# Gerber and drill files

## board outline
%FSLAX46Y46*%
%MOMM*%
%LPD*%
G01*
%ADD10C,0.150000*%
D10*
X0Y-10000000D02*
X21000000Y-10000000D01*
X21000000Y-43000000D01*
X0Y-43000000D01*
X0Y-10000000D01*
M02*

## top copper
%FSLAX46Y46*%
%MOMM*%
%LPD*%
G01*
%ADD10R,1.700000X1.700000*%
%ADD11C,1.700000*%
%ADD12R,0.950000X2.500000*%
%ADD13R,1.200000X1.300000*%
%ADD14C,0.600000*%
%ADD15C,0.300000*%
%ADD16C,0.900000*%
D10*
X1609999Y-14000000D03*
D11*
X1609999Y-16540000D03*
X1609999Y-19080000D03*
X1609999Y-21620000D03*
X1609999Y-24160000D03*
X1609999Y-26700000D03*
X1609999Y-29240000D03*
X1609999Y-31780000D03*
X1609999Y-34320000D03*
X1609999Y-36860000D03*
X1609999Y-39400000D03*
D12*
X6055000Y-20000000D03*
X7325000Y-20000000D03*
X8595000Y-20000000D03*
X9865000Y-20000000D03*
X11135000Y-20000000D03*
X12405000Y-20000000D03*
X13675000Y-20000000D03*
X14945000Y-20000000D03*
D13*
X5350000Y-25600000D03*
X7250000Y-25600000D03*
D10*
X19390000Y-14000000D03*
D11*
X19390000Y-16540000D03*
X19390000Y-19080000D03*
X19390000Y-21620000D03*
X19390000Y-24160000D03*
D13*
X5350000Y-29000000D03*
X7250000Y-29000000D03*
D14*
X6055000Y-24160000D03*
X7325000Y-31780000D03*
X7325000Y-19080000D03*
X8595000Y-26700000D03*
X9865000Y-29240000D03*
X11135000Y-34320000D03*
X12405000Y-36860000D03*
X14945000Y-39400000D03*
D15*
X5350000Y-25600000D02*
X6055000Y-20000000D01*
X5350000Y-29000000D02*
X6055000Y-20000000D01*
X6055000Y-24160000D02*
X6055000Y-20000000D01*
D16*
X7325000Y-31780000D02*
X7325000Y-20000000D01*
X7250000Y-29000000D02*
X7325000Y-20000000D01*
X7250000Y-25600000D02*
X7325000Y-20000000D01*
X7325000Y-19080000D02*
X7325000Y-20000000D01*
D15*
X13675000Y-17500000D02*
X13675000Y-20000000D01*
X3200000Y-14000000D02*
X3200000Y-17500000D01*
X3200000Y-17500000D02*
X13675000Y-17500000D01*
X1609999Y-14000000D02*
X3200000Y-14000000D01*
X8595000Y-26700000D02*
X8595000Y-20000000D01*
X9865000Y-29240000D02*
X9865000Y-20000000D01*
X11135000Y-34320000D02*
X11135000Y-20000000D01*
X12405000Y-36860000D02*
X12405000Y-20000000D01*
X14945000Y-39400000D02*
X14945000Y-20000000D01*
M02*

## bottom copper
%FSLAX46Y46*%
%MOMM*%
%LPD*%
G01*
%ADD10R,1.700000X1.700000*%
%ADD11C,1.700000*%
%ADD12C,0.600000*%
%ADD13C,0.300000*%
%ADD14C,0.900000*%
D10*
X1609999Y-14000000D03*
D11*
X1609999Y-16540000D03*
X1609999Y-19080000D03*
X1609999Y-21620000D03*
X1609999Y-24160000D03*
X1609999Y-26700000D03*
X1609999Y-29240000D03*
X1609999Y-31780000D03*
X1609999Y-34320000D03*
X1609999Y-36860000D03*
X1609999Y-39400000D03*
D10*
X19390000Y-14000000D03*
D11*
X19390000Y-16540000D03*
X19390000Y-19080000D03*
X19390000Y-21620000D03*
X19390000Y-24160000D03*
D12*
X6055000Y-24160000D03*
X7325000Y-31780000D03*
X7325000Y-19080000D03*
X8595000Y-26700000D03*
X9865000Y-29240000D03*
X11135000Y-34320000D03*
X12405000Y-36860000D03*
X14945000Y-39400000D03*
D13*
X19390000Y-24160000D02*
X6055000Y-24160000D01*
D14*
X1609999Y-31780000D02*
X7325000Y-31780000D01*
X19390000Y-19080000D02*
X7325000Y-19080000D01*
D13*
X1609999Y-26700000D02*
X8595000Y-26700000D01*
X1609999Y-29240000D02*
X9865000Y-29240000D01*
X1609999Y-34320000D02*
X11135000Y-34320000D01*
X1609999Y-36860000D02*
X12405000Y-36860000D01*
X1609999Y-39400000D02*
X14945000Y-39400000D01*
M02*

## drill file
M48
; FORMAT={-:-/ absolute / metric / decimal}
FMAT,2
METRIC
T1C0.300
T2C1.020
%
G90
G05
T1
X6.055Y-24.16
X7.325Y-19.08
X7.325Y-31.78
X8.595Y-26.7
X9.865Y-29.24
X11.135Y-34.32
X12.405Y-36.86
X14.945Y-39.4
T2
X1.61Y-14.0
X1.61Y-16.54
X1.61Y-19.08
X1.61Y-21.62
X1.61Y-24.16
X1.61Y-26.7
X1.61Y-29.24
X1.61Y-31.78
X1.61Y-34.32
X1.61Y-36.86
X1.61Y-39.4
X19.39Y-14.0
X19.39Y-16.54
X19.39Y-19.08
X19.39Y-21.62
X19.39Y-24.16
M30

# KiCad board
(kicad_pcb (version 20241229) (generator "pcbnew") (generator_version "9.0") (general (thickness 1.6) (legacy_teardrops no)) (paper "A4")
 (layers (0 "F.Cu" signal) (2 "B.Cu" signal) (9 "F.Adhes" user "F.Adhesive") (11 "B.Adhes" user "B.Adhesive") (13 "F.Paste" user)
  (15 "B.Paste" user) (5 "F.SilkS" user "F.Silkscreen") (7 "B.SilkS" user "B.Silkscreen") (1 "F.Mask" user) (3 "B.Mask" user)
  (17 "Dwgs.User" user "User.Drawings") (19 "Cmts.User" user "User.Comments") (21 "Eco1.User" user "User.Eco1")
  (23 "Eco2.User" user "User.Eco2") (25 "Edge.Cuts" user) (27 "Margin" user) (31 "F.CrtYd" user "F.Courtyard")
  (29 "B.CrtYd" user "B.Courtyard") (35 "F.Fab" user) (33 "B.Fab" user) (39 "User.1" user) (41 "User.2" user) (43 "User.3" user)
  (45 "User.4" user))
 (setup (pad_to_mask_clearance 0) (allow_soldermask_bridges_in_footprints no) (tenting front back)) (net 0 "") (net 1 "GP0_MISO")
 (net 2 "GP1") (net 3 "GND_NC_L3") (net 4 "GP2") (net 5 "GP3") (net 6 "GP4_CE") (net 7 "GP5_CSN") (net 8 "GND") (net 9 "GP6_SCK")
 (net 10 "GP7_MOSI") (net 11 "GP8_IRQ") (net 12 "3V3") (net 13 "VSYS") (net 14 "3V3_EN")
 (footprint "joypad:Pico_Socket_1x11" (layer "F.Cu") (at 1.609999 14)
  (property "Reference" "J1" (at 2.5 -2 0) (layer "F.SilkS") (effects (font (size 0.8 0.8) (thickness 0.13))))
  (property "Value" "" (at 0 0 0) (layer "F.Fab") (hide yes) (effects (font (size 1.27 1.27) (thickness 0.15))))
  (pad "1" thru_hole rect (at 0 0) (size 1.7 1.7) (drill 1.02) (layers "*.Cu" "*.Mask") (remove_unused_layers no) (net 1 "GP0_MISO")
   (thermal_bridge_angle 45))
  (pad "2" thru_hole circle (at 0 2.54) (size 1.7 1.7) (drill 1.02) (layers "*.Cu" "*.Mask") (remove_unused_layers no) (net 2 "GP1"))
  (pad "3" thru_hole circle (at 0 5.08) (size 1.7 1.7) (drill 1.02) (layers "*.Cu" "*.Mask") (remove_unused_layers no) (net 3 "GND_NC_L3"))
  (pad "4" thru_hole circle (at 0 7.62) (size 1.7 1.7) (drill 1.02) (layers "*.Cu" "*.Mask") (remove_unused_layers no) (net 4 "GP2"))
  (pad "5" thru_hole circle (at 0 10.16) (size 1.7 1.7) (drill 1.02) (layers "*.Cu" "*.Mask") (remove_unused_layers no) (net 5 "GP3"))
  (pad "6" thru_hole circle (at 0 12.7) (size 1.7 1.7) (drill 1.02) (layers "*.Cu" "*.Mask") (remove_unused_layers no) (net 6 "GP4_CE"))
  (pad "7" thru_hole circle (at 0 15.24) (size 1.7 1.7) (drill 1.02) (layers "*.Cu" "*.Mask") (remove_unused_layers no) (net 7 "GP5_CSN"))
  (pad "8" thru_hole circle (at 0 17.78) (size 1.7 1.7) (drill 1.02) (layers "*.Cu" "*.Mask") (remove_unused_layers no) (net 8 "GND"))
  (pad "9" thru_hole circle (at 0 20.32) (size 1.7 1.7) (drill 1.02) (layers "*.Cu" "*.Mask") (remove_unused_layers no) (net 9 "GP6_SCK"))
  (pad "10" thru_hole circle (at 0 22.86) (size 1.7 1.7) (drill 1.02) (layers "*.Cu" "*.Mask") (remove_unused_layers no) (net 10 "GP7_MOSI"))
  (pad "11" thru_hole circle (at 0 25.4) (size 1.7 1.7) (drill 1.02) (layers "*.Cu" "*.Mask") (remove_unused_layers no) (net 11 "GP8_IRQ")))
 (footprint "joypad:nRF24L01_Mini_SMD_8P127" (layer "F.Cu") (at 10.5 20)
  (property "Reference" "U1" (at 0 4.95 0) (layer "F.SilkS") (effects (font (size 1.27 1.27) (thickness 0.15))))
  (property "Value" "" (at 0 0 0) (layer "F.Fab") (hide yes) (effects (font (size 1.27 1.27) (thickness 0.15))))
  (pad "1" smd rect (at -4.445 0) (size 0.95 2.5) (layers "F.Cu" "F.Mask" "F.Paste") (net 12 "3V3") (thermal_bridge_angle 45))
  (pad "2" smd rect (at -3.175 0) (size 0.95 2.5) (layers "F.Cu" "F.Mask" "F.Paste") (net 8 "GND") (thermal_bridge_angle 45))
  (pad "3" smd rect (at -1.905 0) (size 0.95 2.5) (layers "F.Cu" "F.Mask" "F.Paste") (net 6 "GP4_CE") (thermal_bridge_angle 45))
  (pad "4" smd rect (at -0.635 0) (size 0.95 2.5) (layers "F.Cu" "F.Mask" "F.Paste") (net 7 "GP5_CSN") (thermal_bridge_angle 45))
  (pad "5" smd rect (at 0.635 0) (size 0.95 2.5) (layers "F.Cu" "F.Mask" "F.Paste") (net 9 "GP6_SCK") (thermal_bridge_angle 45))
  (pad "6" smd rect (at 1.905 0) (size 0.95 2.5) (layers "F.Cu" "F.Mask" "F.Paste") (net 10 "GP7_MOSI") (thermal_bridge_angle 45))
  (pad "7" smd rect (at 3.175 0) (size 0.95 2.5) (layers "F.Cu" "F.Mask" "F.Paste") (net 1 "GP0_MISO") (thermal_bridge_angle 45))
  (pad "8" smd rect (at 4.445 0) (size 0.95 2.5) (layers "F.Cu" "F.Mask" "F.Paste") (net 11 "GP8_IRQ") (thermal_bridge_angle 45))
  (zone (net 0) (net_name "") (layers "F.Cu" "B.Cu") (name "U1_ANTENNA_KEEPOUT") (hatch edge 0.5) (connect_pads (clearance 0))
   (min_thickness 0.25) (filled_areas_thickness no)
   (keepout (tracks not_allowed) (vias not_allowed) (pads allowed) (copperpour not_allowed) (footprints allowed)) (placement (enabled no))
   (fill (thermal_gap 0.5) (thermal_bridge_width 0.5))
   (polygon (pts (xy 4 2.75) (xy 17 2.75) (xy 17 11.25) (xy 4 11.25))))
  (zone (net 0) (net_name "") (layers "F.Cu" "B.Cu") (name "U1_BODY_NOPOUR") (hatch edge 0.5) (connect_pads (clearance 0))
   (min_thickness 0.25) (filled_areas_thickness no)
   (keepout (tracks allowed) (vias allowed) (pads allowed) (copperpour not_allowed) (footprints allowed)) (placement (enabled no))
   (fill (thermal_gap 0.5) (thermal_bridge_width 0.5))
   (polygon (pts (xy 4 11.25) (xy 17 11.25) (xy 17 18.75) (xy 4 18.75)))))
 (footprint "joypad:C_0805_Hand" (layer "F.Cu") (at 6.3 25.6)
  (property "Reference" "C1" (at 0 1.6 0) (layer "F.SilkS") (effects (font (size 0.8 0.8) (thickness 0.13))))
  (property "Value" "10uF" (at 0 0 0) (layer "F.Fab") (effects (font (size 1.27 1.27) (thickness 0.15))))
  (pad "1" smd rect (at -0.95 0) (size 1.2 1.3) (layers "F.Cu" "F.Mask" "F.Paste") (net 12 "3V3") (thermal_bridge_angle 45))
  (pad "2" smd rect (at 0.95 0) (size 1.2 1.3) (layers "F.Cu" "F.Mask" "F.Paste") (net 8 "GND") (thermal_bridge_angle 45)))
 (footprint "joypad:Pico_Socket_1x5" (layer "F.Cu") (at 19.39 14)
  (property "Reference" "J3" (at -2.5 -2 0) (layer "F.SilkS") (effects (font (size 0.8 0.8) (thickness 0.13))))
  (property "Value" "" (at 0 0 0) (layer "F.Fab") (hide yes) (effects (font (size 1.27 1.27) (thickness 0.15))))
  (pad "1" thru_hole rect (at 0 0) (size 1.7 1.7) (drill 1.02) (layers "*.Cu" "*.Mask") (remove_unused_layers no) (thermal_bridge_angle 45))
  (pad "2" thru_hole circle (at 0 2.54) (size 1.7 1.7) (drill 1.02) (layers "*.Cu" "*.Mask") (remove_unused_layers no) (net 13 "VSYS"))
  (pad "3" thru_hole circle (at 0 5.08) (size 1.7 1.7) (drill 1.02) (layers "*.Cu" "*.Mask") (remove_unused_layers no) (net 8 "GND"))
  (pad "4" thru_hole circle (at 0 7.62) (size 1.7 1.7) (drill 1.02) (layers "*.Cu" "*.Mask") (remove_unused_layers no) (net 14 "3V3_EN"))
  (pad "5" thru_hole circle (at 0 10.16) (size 1.7 1.7) (drill 1.02) (layers "*.Cu" "*.Mask") (remove_unused_layers no) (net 12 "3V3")))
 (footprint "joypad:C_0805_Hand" (layer "F.Cu") (at 6.3 29)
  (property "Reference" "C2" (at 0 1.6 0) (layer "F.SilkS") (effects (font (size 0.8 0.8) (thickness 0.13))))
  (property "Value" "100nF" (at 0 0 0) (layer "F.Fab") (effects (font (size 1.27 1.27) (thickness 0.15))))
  (pad "1" smd rect (at -0.95 0) (size 1.2 1.3) (layers "F.Cu" "F.Mask" "F.Paste") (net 12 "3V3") (thermal_bridge_angle 45))
  (pad "2" smd rect (at 0.95 0) (size 1.2 1.3) (layers "F.Cu" "F.Mask" "F.Paste") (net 8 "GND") (thermal_bridge_angle 45)))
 (gr_rect (start 0 10) (end 21 43) (stroke (width 0.15) (type default)) (fill no) (layer "Edge.Cuts"))
 (segment (start 5.35 25.6) (end 6.055 20) (width 0.3) (layer "F.Cu") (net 12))
 (segment (start 5.35 29) (end 6.055 20) (width 0.3) (layer "F.Cu") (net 12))
 (segment (start 6.055 24.16) (end 6.055 20) (width 0.3) (layer "F.Cu") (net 12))
 (via (at 6.055 24.16) (size 0.6) (drill 0.3) (layers "F.Cu" "B.Cu") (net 12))
 (segment (start 19.39 24.16) (end 6.055 24.16) (width 0.3) (layer "B.Cu") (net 12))
 (segment (start 7.325 31.78) (end 7.325 20) (width 0.9) (layer "F.Cu") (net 8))
 (segment (start 7.25 29) (end 7.325 20) (width 0.9) (layer "F.Cu") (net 8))
 (segment (start 7.25 25.6) (end 7.325 20) (width 0.9) (layer "F.Cu") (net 8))
 (segment (start 7.325 19.08) (end 7.325 20) (width 0.9) (layer "F.Cu") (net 8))
 (via (at 7.325 31.78) (size 0.6) (drill 0.3) (layers "F.Cu" "B.Cu") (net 8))
 (via (at 7.325 19.08) (size 0.6) (drill 0.3) (layers "F.Cu" "B.Cu") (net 8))
 (segment (start 1.609999 31.78) (end 7.325 31.78) (width 0.9) (layer "B.Cu") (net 8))
 (segment (start 19.39 19.08) (end 7.325 19.08) (width 0.9) (layer "B.Cu") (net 8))
 (segment (start 13.675 17.5) (end 13.675 20) (width 0.3) (layer "F.Cu") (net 1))
 (segment (start 3.2 14) (end 3.2 17.5) (width 0.3) (layer "F.Cu") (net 1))
 (segment (start 3.2 17.5) (end 13.675 17.5) (width 0.3) (layer "F.Cu") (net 1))
 (segment (start 1.609999 14) (end 3.2 14) (width 0.3) (layer "F.Cu") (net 1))
 (segment (start 8.595 26.7) (end 8.595 20) (width 0.3) (layer "F.Cu") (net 6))
 (via (at 8.595 26.7) (size 0.6) (drill 0.3) (layers "F.Cu" "B.Cu") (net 6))
 (segment (start 1.609999 26.7) (end 8.595 26.7) (width 0.3) (layer "B.Cu") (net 6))
 (segment (start 9.865 29.24) (end 9.865 20) (width 0.3) (layer "F.Cu") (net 7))
 (via (at 9.865 29.24) (size 0.6) (drill 0.3) (layers "F.Cu" "B.Cu") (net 7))
 (segment (start 1.609999 29.24) (end 9.865 29.24) (width 0.3) (layer "B.Cu") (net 7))
 (segment (start 11.135 34.32) (end 11.135 20) (width 0.3) (layer "F.Cu") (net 9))
 (via (at 11.135 34.32) (size 0.6) (drill 0.3) (layers "F.Cu" "B.Cu") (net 9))
 (segment (start 1.609999 34.32) (end 11.135 34.32) (width 0.3) (layer "B.Cu") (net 9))
 (segment (start 12.405 36.86) (end 12.405 20) (width 0.3) (layer "F.Cu") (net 10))
 (via (at 12.405 36.86) (size 0.6) (drill 0.3) (layers "F.Cu" "B.Cu") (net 10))
 (segment (start 1.609999 36.86) (end 12.405 36.86) (width 0.3) (layer "B.Cu") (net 10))
 (segment (start 14.945 39.4) (end 14.945 20) (width 0.3) (layer "F.Cu") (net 11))
 (via (at 14.945 39.4) (size 0.6) (drill 0.3) (layers "F.Cu" "B.Cu") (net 11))
 (segment (start 1.609999 39.4) (end 14.945 39.4) (width 0.3) (layer "B.Cu") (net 11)))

